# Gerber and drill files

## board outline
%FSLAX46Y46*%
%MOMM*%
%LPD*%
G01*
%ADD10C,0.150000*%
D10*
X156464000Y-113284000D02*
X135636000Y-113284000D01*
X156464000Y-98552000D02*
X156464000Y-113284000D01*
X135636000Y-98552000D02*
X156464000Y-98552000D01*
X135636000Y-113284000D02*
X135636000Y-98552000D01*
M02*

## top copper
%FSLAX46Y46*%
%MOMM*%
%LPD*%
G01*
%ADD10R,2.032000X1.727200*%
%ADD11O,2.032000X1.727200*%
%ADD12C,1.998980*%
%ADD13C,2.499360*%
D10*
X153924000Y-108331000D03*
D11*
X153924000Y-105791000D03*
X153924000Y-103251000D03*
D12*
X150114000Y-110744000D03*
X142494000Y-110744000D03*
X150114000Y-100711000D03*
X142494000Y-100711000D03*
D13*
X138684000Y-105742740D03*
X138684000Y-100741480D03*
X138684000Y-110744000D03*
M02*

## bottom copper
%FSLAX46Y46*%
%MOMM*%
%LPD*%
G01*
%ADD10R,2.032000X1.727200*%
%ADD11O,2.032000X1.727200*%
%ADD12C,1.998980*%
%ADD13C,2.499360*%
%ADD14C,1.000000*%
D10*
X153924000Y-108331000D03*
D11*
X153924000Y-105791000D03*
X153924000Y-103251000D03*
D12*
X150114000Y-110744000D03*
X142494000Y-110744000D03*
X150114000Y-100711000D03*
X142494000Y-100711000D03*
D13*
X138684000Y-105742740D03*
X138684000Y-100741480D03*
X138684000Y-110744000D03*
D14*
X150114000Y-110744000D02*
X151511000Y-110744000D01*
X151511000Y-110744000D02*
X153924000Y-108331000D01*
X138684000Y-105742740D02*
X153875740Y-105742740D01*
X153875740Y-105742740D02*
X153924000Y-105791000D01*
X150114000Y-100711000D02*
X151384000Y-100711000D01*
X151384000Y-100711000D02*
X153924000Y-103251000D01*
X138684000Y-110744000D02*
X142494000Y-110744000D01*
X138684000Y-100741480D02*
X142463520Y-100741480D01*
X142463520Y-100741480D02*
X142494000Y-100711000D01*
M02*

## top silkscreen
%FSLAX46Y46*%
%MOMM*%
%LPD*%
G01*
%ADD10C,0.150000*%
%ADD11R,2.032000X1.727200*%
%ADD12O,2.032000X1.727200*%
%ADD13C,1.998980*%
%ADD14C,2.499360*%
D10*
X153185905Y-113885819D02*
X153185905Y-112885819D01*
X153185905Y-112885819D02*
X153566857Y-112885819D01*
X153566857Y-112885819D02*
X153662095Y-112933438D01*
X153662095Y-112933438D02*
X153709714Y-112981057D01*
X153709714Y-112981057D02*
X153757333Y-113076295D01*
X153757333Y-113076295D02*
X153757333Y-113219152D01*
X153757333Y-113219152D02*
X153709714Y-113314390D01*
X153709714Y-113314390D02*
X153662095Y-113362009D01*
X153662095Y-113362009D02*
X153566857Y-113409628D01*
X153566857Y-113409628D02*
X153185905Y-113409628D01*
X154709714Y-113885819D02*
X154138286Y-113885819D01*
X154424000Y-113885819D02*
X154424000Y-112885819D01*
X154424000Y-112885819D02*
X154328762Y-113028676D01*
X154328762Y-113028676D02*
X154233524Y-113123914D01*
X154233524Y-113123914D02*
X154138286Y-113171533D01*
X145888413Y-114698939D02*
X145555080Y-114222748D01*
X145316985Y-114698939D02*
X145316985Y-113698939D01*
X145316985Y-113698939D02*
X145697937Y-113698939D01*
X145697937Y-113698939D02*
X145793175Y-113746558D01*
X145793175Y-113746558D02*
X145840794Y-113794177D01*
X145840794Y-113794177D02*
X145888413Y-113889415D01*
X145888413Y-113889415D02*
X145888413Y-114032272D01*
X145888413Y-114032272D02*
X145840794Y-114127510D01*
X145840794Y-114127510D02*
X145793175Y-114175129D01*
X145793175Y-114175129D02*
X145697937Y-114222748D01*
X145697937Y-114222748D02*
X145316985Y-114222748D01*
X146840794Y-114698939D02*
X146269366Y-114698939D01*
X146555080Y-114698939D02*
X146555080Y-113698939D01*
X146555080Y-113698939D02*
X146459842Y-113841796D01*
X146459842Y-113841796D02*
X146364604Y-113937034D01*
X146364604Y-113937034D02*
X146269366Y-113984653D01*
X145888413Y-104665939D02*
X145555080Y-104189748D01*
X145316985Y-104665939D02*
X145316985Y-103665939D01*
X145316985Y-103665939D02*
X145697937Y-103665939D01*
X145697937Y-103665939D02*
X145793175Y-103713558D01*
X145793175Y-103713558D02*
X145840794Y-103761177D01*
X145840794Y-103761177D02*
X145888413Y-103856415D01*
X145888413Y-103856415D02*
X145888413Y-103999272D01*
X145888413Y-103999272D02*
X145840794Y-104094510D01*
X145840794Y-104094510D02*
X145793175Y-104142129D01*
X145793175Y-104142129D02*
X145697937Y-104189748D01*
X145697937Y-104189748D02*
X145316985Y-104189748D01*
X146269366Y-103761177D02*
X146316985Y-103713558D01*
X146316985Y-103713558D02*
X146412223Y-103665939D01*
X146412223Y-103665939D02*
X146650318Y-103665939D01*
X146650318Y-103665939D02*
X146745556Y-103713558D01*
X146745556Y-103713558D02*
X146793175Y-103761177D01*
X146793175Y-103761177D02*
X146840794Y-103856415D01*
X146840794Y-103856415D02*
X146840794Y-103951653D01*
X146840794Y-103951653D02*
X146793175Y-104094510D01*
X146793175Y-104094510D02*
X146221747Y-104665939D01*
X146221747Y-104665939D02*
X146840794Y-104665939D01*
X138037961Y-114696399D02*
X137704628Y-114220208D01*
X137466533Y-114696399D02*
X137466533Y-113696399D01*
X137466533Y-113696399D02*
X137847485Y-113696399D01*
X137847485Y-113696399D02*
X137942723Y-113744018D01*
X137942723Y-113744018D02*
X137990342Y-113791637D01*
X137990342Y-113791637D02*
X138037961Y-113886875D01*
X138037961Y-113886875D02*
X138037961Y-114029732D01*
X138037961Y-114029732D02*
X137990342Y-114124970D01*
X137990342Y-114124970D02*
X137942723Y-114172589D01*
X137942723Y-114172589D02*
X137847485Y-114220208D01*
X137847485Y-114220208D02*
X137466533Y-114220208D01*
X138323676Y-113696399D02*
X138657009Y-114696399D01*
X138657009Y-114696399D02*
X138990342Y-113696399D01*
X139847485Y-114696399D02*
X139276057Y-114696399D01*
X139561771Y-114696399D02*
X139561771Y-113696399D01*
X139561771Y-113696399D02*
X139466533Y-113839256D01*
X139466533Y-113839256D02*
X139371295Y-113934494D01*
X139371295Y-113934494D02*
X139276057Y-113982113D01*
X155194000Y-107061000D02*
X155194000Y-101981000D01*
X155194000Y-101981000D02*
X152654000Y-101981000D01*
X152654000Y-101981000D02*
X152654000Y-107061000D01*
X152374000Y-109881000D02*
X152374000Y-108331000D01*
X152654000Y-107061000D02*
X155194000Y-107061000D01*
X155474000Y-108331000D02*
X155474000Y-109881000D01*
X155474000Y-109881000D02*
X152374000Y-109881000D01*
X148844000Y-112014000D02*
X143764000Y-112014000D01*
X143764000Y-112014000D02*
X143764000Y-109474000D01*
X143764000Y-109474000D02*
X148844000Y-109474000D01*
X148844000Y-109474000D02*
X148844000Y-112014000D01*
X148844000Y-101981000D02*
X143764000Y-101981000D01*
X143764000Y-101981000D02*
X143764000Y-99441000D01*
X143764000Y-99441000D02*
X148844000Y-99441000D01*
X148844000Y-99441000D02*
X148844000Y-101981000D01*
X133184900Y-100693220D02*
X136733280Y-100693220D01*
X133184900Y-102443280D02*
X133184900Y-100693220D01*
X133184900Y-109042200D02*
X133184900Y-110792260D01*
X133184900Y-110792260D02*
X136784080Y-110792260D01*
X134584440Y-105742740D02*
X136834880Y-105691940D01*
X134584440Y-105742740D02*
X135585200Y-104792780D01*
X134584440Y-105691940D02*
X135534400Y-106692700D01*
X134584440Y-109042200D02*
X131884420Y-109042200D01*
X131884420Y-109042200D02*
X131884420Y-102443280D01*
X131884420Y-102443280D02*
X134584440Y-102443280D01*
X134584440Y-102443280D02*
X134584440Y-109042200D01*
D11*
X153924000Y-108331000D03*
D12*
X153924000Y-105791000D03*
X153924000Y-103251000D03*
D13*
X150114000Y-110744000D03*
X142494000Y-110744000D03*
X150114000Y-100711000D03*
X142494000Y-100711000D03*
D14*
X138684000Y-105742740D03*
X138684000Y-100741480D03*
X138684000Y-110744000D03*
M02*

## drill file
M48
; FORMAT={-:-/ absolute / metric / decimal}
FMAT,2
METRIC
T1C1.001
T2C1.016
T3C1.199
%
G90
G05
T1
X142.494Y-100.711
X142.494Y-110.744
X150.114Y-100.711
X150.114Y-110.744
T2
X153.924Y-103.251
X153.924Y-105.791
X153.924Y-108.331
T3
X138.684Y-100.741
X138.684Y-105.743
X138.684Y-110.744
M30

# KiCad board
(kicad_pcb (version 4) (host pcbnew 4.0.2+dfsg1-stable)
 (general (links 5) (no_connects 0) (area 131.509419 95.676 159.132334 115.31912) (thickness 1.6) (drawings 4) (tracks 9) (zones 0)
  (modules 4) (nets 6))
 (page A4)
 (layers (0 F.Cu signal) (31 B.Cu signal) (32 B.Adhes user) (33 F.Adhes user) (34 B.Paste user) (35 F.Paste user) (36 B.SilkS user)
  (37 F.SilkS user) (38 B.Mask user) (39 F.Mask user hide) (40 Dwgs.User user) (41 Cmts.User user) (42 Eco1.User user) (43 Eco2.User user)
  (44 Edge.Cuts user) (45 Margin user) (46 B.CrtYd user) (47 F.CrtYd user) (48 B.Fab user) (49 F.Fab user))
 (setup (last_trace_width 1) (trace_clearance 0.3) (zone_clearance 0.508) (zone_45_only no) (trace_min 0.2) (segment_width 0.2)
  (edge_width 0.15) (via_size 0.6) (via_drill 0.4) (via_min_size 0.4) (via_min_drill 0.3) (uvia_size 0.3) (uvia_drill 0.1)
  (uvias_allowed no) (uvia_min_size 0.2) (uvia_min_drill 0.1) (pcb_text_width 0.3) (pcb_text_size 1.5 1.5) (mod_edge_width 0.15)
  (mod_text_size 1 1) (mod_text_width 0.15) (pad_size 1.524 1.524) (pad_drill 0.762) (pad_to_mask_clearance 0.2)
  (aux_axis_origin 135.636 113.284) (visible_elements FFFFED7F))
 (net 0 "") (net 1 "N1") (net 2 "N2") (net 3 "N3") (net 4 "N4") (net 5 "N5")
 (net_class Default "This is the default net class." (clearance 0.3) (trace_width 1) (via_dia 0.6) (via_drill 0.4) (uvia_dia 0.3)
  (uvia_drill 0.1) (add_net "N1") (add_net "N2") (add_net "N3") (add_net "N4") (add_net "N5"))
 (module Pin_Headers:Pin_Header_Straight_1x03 (layer F.Cu) (at 153.924 108.331 180)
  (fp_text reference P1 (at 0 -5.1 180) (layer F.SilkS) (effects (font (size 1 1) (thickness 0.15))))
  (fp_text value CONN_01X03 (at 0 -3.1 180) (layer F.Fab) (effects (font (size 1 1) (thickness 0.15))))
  (fp_line (start -1.27 1.27) (end -1.27 6.35) (layer F.SilkS) (width 0.15))
  (fp_line (start -1.27 6.35) (end 1.27 6.35) (layer F.SilkS) (width 0.15))
  (fp_line (start 1.27 6.35) (end 1.27 1.27) (layer F.SilkS) (width 0.15))
  (fp_line (start 1.55 -1.55) (end 1.55 0) (layer F.SilkS) (width 0.15))
  (fp_line (start 1.27 1.27) (end -1.27 1.27) (layer F.SilkS) (width 0.15))
  (fp_line (start -1.55 0) (end -1.55 -1.55) (layer F.SilkS) (width 0.15))
  (fp_line (start -1.55 -1.55) (end 1.55 -1.55) (layer F.SilkS) (width 0.15))
  (pad 1 thru_hole rect (at 0 0 180) (size 2.032 1.7272) (drill 1.016) (layers *.Cu *.Mask F.SilkS) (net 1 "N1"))
  (pad 2 thru_hole oval (at 0 2.54 180) (size 2.032 1.7272) (drill 1.016) (layers *.Cu *.Mask F.SilkS) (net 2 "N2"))
  (pad 3 thru_hole oval (at 0 5.08 180) (size 2.032 1.7272) (drill 1.016) (layers *.Cu *.Mask F.SilkS) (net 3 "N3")))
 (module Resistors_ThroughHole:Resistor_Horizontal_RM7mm (layer F.Cu) (at 150.114 110.744 180)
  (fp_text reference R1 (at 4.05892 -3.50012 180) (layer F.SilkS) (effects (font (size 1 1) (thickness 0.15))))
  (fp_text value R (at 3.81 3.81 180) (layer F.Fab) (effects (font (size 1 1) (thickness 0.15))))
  (fp_line (start 1.27 -1.27) (end 6.35 -1.27) (layer F.SilkS) (width 0.15))
  (fp_line (start 6.35 -1.27) (end 6.35 1.27) (layer F.SilkS) (width 0.15))
  (fp_line (start 6.35 1.27) (end 1.27 1.27) (layer F.SilkS) (width 0.15))
  (fp_line (start 1.27 1.27) (end 1.27 -1.27) (layer F.SilkS) (width 0.15))
  (pad 1 thru_hole circle (at 0 0 180) (size 1.99898 1.99898) (drill 1.00076) (layers *.Cu *.SilkS *.Mask) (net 1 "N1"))
  (pad 2 thru_hole circle (at 7.62 0 180) (size 1.99898 1.99898) (drill 1.00076) (layers *.Cu *.SilkS *.Mask) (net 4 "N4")))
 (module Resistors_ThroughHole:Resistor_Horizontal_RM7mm (layer F.Cu) (at 150.114 100.711 180)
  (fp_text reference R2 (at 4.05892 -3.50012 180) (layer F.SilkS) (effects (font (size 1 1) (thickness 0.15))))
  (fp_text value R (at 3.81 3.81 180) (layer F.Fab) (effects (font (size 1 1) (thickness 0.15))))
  (fp_line (start 1.27 -1.27) (end 6.35 -1.27) (layer F.SilkS) (width 0.15))
  (fp_line (start 6.35 -1.27) (end 6.35 1.27) (layer F.SilkS) (width 0.15))
  (fp_line (start 6.35 1.27) (end 1.27 1.27) (layer F.SilkS) (width 0.15))
  (fp_line (start 1.27 1.27) (end 1.27 -1.27) (layer F.SilkS) (width 0.15))
  (pad 1 thru_hole circle (at 0 0 180) (size 1.99898 1.99898) (drill 1.00076) (layers *.Cu *.SilkS *.Mask) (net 3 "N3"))
  (pad 2 thru_hole circle (at 7.62 0 180) (size 1.99898 1.99898) (drill 1.00076) (layers *.Cu *.SilkS *.Mask) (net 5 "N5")))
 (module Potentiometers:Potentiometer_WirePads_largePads (layer F.Cu) (at 138.684 110.744 180)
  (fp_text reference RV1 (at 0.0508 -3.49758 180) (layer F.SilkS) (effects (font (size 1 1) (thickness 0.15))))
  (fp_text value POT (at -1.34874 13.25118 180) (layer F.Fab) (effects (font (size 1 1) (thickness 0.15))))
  (fp_line (start 5.4991 10.05078) (end 1.95072 10.05078) (layer F.SilkS) (width 0.15))
  (fp_line (start 5.4991 8.30072) (end 5.4991 10.05078) (layer F.SilkS) (width 0.15))
  (fp_line (start 5.4991 1.7018) (end 5.4991 -0.04826) (layer F.SilkS) (width 0.15))
  (fp_line (start 5.4991 -0.04826) (end 1.89992 -0.04826) (layer F.SilkS) (width 0.15))
  (fp_line (start 4.09956 5.00126) (end 1.84912 5.05206) (layer F.SilkS) (width 0.15))
  (fp_line (start 4.09956 5.00126) (end 3.0988 5.95122) (layer F.SilkS) (width 0.15))
  (fp_line (start 4.09956 5.05206) (end 3.1496 4.0513) (layer F.SilkS) (width 0.15))
  (fp_line (start 4.09956 1.7018) (end 6.79958 1.7018) (layer F.SilkS) (width 0.15))
  (fp_line (start 6.79958 1.7018) (end 6.79958 8.30072) (layer F.SilkS) (width 0.15))
  (fp_line (start 6.79958 8.30072) (end 4.09956 8.30072) (layer F.SilkS) (width 0.15))
  (fp_line (start 4.09956 8.30072) (end 4.09956 1.7018) (layer F.SilkS) (width 0.15))
  (pad 2 thru_hole circle (at 0 5.00126 180) (size 2.49936 2.49936) (drill 1.19888) (layers *.Cu *.Mask F.SilkS) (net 2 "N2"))
  (pad 3 thru_hole circle (at 0 10.00252 180) (size 2.49936 2.49936) (drill 1.19888) (layers *.Cu *.Mask F.SilkS) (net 5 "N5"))
  (pad 1 thru_hole circle (at 0 0 180) (size 2.49936 2.49936) (drill 1.19888) (layers *.Cu *.Mask F.SilkS) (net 4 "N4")))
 (gr_line (start 156.464 113.284) (end 135.636 113.284) (angle 90) (layer Edge.Cuts) (width 0.15))
 (gr_line (start 156.464 98.552) (end 156.464 113.284) (angle 90) (layer Edge.Cuts) (width 0.15))
 (gr_line (start 135.636 98.552) (end 156.464 98.552) (angle 90) (layer Edge.Cuts) (width 0.15))
 (gr_line (start 135.636 113.284) (end 135.636 98.552) (angle 90) (layer Edge.Cuts) (width 0.15))
 (segment (start 150.114 110.744) (end 151.511 110.744) (width 1) (layer B.Cu) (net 1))
 (segment (start 151.511 110.744) (end 153.924 108.331) (width 1) (layer B.Cu) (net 1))
 (segment (start 138.684 105.74274) (end 153.87574 105.74274) (width 1) (layer B.Cu) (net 2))
 (segment (start 153.87574 105.74274) (end 153.924 105.791) (width 1) (layer B.Cu) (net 2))
 (segment (start 150.114 100.711) (end 151.384 100.711) (width 1) (layer B.Cu) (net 3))
 (segment (start 151.384 100.711) (end 153.924 103.251) (width 1) (layer B.Cu) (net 3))
 (segment (start 138.684 110.744) (end 142.494 110.744) (width 1) (layer B.Cu) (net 4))
 (segment (start 138.684 100.74148) (end 142.46352 100.74148) (width 1) (layer B.Cu) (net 5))
 (segment (start 142.46352 100.74148) (end 142.494 100.711) (width 1) (layer B.Cu) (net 5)))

